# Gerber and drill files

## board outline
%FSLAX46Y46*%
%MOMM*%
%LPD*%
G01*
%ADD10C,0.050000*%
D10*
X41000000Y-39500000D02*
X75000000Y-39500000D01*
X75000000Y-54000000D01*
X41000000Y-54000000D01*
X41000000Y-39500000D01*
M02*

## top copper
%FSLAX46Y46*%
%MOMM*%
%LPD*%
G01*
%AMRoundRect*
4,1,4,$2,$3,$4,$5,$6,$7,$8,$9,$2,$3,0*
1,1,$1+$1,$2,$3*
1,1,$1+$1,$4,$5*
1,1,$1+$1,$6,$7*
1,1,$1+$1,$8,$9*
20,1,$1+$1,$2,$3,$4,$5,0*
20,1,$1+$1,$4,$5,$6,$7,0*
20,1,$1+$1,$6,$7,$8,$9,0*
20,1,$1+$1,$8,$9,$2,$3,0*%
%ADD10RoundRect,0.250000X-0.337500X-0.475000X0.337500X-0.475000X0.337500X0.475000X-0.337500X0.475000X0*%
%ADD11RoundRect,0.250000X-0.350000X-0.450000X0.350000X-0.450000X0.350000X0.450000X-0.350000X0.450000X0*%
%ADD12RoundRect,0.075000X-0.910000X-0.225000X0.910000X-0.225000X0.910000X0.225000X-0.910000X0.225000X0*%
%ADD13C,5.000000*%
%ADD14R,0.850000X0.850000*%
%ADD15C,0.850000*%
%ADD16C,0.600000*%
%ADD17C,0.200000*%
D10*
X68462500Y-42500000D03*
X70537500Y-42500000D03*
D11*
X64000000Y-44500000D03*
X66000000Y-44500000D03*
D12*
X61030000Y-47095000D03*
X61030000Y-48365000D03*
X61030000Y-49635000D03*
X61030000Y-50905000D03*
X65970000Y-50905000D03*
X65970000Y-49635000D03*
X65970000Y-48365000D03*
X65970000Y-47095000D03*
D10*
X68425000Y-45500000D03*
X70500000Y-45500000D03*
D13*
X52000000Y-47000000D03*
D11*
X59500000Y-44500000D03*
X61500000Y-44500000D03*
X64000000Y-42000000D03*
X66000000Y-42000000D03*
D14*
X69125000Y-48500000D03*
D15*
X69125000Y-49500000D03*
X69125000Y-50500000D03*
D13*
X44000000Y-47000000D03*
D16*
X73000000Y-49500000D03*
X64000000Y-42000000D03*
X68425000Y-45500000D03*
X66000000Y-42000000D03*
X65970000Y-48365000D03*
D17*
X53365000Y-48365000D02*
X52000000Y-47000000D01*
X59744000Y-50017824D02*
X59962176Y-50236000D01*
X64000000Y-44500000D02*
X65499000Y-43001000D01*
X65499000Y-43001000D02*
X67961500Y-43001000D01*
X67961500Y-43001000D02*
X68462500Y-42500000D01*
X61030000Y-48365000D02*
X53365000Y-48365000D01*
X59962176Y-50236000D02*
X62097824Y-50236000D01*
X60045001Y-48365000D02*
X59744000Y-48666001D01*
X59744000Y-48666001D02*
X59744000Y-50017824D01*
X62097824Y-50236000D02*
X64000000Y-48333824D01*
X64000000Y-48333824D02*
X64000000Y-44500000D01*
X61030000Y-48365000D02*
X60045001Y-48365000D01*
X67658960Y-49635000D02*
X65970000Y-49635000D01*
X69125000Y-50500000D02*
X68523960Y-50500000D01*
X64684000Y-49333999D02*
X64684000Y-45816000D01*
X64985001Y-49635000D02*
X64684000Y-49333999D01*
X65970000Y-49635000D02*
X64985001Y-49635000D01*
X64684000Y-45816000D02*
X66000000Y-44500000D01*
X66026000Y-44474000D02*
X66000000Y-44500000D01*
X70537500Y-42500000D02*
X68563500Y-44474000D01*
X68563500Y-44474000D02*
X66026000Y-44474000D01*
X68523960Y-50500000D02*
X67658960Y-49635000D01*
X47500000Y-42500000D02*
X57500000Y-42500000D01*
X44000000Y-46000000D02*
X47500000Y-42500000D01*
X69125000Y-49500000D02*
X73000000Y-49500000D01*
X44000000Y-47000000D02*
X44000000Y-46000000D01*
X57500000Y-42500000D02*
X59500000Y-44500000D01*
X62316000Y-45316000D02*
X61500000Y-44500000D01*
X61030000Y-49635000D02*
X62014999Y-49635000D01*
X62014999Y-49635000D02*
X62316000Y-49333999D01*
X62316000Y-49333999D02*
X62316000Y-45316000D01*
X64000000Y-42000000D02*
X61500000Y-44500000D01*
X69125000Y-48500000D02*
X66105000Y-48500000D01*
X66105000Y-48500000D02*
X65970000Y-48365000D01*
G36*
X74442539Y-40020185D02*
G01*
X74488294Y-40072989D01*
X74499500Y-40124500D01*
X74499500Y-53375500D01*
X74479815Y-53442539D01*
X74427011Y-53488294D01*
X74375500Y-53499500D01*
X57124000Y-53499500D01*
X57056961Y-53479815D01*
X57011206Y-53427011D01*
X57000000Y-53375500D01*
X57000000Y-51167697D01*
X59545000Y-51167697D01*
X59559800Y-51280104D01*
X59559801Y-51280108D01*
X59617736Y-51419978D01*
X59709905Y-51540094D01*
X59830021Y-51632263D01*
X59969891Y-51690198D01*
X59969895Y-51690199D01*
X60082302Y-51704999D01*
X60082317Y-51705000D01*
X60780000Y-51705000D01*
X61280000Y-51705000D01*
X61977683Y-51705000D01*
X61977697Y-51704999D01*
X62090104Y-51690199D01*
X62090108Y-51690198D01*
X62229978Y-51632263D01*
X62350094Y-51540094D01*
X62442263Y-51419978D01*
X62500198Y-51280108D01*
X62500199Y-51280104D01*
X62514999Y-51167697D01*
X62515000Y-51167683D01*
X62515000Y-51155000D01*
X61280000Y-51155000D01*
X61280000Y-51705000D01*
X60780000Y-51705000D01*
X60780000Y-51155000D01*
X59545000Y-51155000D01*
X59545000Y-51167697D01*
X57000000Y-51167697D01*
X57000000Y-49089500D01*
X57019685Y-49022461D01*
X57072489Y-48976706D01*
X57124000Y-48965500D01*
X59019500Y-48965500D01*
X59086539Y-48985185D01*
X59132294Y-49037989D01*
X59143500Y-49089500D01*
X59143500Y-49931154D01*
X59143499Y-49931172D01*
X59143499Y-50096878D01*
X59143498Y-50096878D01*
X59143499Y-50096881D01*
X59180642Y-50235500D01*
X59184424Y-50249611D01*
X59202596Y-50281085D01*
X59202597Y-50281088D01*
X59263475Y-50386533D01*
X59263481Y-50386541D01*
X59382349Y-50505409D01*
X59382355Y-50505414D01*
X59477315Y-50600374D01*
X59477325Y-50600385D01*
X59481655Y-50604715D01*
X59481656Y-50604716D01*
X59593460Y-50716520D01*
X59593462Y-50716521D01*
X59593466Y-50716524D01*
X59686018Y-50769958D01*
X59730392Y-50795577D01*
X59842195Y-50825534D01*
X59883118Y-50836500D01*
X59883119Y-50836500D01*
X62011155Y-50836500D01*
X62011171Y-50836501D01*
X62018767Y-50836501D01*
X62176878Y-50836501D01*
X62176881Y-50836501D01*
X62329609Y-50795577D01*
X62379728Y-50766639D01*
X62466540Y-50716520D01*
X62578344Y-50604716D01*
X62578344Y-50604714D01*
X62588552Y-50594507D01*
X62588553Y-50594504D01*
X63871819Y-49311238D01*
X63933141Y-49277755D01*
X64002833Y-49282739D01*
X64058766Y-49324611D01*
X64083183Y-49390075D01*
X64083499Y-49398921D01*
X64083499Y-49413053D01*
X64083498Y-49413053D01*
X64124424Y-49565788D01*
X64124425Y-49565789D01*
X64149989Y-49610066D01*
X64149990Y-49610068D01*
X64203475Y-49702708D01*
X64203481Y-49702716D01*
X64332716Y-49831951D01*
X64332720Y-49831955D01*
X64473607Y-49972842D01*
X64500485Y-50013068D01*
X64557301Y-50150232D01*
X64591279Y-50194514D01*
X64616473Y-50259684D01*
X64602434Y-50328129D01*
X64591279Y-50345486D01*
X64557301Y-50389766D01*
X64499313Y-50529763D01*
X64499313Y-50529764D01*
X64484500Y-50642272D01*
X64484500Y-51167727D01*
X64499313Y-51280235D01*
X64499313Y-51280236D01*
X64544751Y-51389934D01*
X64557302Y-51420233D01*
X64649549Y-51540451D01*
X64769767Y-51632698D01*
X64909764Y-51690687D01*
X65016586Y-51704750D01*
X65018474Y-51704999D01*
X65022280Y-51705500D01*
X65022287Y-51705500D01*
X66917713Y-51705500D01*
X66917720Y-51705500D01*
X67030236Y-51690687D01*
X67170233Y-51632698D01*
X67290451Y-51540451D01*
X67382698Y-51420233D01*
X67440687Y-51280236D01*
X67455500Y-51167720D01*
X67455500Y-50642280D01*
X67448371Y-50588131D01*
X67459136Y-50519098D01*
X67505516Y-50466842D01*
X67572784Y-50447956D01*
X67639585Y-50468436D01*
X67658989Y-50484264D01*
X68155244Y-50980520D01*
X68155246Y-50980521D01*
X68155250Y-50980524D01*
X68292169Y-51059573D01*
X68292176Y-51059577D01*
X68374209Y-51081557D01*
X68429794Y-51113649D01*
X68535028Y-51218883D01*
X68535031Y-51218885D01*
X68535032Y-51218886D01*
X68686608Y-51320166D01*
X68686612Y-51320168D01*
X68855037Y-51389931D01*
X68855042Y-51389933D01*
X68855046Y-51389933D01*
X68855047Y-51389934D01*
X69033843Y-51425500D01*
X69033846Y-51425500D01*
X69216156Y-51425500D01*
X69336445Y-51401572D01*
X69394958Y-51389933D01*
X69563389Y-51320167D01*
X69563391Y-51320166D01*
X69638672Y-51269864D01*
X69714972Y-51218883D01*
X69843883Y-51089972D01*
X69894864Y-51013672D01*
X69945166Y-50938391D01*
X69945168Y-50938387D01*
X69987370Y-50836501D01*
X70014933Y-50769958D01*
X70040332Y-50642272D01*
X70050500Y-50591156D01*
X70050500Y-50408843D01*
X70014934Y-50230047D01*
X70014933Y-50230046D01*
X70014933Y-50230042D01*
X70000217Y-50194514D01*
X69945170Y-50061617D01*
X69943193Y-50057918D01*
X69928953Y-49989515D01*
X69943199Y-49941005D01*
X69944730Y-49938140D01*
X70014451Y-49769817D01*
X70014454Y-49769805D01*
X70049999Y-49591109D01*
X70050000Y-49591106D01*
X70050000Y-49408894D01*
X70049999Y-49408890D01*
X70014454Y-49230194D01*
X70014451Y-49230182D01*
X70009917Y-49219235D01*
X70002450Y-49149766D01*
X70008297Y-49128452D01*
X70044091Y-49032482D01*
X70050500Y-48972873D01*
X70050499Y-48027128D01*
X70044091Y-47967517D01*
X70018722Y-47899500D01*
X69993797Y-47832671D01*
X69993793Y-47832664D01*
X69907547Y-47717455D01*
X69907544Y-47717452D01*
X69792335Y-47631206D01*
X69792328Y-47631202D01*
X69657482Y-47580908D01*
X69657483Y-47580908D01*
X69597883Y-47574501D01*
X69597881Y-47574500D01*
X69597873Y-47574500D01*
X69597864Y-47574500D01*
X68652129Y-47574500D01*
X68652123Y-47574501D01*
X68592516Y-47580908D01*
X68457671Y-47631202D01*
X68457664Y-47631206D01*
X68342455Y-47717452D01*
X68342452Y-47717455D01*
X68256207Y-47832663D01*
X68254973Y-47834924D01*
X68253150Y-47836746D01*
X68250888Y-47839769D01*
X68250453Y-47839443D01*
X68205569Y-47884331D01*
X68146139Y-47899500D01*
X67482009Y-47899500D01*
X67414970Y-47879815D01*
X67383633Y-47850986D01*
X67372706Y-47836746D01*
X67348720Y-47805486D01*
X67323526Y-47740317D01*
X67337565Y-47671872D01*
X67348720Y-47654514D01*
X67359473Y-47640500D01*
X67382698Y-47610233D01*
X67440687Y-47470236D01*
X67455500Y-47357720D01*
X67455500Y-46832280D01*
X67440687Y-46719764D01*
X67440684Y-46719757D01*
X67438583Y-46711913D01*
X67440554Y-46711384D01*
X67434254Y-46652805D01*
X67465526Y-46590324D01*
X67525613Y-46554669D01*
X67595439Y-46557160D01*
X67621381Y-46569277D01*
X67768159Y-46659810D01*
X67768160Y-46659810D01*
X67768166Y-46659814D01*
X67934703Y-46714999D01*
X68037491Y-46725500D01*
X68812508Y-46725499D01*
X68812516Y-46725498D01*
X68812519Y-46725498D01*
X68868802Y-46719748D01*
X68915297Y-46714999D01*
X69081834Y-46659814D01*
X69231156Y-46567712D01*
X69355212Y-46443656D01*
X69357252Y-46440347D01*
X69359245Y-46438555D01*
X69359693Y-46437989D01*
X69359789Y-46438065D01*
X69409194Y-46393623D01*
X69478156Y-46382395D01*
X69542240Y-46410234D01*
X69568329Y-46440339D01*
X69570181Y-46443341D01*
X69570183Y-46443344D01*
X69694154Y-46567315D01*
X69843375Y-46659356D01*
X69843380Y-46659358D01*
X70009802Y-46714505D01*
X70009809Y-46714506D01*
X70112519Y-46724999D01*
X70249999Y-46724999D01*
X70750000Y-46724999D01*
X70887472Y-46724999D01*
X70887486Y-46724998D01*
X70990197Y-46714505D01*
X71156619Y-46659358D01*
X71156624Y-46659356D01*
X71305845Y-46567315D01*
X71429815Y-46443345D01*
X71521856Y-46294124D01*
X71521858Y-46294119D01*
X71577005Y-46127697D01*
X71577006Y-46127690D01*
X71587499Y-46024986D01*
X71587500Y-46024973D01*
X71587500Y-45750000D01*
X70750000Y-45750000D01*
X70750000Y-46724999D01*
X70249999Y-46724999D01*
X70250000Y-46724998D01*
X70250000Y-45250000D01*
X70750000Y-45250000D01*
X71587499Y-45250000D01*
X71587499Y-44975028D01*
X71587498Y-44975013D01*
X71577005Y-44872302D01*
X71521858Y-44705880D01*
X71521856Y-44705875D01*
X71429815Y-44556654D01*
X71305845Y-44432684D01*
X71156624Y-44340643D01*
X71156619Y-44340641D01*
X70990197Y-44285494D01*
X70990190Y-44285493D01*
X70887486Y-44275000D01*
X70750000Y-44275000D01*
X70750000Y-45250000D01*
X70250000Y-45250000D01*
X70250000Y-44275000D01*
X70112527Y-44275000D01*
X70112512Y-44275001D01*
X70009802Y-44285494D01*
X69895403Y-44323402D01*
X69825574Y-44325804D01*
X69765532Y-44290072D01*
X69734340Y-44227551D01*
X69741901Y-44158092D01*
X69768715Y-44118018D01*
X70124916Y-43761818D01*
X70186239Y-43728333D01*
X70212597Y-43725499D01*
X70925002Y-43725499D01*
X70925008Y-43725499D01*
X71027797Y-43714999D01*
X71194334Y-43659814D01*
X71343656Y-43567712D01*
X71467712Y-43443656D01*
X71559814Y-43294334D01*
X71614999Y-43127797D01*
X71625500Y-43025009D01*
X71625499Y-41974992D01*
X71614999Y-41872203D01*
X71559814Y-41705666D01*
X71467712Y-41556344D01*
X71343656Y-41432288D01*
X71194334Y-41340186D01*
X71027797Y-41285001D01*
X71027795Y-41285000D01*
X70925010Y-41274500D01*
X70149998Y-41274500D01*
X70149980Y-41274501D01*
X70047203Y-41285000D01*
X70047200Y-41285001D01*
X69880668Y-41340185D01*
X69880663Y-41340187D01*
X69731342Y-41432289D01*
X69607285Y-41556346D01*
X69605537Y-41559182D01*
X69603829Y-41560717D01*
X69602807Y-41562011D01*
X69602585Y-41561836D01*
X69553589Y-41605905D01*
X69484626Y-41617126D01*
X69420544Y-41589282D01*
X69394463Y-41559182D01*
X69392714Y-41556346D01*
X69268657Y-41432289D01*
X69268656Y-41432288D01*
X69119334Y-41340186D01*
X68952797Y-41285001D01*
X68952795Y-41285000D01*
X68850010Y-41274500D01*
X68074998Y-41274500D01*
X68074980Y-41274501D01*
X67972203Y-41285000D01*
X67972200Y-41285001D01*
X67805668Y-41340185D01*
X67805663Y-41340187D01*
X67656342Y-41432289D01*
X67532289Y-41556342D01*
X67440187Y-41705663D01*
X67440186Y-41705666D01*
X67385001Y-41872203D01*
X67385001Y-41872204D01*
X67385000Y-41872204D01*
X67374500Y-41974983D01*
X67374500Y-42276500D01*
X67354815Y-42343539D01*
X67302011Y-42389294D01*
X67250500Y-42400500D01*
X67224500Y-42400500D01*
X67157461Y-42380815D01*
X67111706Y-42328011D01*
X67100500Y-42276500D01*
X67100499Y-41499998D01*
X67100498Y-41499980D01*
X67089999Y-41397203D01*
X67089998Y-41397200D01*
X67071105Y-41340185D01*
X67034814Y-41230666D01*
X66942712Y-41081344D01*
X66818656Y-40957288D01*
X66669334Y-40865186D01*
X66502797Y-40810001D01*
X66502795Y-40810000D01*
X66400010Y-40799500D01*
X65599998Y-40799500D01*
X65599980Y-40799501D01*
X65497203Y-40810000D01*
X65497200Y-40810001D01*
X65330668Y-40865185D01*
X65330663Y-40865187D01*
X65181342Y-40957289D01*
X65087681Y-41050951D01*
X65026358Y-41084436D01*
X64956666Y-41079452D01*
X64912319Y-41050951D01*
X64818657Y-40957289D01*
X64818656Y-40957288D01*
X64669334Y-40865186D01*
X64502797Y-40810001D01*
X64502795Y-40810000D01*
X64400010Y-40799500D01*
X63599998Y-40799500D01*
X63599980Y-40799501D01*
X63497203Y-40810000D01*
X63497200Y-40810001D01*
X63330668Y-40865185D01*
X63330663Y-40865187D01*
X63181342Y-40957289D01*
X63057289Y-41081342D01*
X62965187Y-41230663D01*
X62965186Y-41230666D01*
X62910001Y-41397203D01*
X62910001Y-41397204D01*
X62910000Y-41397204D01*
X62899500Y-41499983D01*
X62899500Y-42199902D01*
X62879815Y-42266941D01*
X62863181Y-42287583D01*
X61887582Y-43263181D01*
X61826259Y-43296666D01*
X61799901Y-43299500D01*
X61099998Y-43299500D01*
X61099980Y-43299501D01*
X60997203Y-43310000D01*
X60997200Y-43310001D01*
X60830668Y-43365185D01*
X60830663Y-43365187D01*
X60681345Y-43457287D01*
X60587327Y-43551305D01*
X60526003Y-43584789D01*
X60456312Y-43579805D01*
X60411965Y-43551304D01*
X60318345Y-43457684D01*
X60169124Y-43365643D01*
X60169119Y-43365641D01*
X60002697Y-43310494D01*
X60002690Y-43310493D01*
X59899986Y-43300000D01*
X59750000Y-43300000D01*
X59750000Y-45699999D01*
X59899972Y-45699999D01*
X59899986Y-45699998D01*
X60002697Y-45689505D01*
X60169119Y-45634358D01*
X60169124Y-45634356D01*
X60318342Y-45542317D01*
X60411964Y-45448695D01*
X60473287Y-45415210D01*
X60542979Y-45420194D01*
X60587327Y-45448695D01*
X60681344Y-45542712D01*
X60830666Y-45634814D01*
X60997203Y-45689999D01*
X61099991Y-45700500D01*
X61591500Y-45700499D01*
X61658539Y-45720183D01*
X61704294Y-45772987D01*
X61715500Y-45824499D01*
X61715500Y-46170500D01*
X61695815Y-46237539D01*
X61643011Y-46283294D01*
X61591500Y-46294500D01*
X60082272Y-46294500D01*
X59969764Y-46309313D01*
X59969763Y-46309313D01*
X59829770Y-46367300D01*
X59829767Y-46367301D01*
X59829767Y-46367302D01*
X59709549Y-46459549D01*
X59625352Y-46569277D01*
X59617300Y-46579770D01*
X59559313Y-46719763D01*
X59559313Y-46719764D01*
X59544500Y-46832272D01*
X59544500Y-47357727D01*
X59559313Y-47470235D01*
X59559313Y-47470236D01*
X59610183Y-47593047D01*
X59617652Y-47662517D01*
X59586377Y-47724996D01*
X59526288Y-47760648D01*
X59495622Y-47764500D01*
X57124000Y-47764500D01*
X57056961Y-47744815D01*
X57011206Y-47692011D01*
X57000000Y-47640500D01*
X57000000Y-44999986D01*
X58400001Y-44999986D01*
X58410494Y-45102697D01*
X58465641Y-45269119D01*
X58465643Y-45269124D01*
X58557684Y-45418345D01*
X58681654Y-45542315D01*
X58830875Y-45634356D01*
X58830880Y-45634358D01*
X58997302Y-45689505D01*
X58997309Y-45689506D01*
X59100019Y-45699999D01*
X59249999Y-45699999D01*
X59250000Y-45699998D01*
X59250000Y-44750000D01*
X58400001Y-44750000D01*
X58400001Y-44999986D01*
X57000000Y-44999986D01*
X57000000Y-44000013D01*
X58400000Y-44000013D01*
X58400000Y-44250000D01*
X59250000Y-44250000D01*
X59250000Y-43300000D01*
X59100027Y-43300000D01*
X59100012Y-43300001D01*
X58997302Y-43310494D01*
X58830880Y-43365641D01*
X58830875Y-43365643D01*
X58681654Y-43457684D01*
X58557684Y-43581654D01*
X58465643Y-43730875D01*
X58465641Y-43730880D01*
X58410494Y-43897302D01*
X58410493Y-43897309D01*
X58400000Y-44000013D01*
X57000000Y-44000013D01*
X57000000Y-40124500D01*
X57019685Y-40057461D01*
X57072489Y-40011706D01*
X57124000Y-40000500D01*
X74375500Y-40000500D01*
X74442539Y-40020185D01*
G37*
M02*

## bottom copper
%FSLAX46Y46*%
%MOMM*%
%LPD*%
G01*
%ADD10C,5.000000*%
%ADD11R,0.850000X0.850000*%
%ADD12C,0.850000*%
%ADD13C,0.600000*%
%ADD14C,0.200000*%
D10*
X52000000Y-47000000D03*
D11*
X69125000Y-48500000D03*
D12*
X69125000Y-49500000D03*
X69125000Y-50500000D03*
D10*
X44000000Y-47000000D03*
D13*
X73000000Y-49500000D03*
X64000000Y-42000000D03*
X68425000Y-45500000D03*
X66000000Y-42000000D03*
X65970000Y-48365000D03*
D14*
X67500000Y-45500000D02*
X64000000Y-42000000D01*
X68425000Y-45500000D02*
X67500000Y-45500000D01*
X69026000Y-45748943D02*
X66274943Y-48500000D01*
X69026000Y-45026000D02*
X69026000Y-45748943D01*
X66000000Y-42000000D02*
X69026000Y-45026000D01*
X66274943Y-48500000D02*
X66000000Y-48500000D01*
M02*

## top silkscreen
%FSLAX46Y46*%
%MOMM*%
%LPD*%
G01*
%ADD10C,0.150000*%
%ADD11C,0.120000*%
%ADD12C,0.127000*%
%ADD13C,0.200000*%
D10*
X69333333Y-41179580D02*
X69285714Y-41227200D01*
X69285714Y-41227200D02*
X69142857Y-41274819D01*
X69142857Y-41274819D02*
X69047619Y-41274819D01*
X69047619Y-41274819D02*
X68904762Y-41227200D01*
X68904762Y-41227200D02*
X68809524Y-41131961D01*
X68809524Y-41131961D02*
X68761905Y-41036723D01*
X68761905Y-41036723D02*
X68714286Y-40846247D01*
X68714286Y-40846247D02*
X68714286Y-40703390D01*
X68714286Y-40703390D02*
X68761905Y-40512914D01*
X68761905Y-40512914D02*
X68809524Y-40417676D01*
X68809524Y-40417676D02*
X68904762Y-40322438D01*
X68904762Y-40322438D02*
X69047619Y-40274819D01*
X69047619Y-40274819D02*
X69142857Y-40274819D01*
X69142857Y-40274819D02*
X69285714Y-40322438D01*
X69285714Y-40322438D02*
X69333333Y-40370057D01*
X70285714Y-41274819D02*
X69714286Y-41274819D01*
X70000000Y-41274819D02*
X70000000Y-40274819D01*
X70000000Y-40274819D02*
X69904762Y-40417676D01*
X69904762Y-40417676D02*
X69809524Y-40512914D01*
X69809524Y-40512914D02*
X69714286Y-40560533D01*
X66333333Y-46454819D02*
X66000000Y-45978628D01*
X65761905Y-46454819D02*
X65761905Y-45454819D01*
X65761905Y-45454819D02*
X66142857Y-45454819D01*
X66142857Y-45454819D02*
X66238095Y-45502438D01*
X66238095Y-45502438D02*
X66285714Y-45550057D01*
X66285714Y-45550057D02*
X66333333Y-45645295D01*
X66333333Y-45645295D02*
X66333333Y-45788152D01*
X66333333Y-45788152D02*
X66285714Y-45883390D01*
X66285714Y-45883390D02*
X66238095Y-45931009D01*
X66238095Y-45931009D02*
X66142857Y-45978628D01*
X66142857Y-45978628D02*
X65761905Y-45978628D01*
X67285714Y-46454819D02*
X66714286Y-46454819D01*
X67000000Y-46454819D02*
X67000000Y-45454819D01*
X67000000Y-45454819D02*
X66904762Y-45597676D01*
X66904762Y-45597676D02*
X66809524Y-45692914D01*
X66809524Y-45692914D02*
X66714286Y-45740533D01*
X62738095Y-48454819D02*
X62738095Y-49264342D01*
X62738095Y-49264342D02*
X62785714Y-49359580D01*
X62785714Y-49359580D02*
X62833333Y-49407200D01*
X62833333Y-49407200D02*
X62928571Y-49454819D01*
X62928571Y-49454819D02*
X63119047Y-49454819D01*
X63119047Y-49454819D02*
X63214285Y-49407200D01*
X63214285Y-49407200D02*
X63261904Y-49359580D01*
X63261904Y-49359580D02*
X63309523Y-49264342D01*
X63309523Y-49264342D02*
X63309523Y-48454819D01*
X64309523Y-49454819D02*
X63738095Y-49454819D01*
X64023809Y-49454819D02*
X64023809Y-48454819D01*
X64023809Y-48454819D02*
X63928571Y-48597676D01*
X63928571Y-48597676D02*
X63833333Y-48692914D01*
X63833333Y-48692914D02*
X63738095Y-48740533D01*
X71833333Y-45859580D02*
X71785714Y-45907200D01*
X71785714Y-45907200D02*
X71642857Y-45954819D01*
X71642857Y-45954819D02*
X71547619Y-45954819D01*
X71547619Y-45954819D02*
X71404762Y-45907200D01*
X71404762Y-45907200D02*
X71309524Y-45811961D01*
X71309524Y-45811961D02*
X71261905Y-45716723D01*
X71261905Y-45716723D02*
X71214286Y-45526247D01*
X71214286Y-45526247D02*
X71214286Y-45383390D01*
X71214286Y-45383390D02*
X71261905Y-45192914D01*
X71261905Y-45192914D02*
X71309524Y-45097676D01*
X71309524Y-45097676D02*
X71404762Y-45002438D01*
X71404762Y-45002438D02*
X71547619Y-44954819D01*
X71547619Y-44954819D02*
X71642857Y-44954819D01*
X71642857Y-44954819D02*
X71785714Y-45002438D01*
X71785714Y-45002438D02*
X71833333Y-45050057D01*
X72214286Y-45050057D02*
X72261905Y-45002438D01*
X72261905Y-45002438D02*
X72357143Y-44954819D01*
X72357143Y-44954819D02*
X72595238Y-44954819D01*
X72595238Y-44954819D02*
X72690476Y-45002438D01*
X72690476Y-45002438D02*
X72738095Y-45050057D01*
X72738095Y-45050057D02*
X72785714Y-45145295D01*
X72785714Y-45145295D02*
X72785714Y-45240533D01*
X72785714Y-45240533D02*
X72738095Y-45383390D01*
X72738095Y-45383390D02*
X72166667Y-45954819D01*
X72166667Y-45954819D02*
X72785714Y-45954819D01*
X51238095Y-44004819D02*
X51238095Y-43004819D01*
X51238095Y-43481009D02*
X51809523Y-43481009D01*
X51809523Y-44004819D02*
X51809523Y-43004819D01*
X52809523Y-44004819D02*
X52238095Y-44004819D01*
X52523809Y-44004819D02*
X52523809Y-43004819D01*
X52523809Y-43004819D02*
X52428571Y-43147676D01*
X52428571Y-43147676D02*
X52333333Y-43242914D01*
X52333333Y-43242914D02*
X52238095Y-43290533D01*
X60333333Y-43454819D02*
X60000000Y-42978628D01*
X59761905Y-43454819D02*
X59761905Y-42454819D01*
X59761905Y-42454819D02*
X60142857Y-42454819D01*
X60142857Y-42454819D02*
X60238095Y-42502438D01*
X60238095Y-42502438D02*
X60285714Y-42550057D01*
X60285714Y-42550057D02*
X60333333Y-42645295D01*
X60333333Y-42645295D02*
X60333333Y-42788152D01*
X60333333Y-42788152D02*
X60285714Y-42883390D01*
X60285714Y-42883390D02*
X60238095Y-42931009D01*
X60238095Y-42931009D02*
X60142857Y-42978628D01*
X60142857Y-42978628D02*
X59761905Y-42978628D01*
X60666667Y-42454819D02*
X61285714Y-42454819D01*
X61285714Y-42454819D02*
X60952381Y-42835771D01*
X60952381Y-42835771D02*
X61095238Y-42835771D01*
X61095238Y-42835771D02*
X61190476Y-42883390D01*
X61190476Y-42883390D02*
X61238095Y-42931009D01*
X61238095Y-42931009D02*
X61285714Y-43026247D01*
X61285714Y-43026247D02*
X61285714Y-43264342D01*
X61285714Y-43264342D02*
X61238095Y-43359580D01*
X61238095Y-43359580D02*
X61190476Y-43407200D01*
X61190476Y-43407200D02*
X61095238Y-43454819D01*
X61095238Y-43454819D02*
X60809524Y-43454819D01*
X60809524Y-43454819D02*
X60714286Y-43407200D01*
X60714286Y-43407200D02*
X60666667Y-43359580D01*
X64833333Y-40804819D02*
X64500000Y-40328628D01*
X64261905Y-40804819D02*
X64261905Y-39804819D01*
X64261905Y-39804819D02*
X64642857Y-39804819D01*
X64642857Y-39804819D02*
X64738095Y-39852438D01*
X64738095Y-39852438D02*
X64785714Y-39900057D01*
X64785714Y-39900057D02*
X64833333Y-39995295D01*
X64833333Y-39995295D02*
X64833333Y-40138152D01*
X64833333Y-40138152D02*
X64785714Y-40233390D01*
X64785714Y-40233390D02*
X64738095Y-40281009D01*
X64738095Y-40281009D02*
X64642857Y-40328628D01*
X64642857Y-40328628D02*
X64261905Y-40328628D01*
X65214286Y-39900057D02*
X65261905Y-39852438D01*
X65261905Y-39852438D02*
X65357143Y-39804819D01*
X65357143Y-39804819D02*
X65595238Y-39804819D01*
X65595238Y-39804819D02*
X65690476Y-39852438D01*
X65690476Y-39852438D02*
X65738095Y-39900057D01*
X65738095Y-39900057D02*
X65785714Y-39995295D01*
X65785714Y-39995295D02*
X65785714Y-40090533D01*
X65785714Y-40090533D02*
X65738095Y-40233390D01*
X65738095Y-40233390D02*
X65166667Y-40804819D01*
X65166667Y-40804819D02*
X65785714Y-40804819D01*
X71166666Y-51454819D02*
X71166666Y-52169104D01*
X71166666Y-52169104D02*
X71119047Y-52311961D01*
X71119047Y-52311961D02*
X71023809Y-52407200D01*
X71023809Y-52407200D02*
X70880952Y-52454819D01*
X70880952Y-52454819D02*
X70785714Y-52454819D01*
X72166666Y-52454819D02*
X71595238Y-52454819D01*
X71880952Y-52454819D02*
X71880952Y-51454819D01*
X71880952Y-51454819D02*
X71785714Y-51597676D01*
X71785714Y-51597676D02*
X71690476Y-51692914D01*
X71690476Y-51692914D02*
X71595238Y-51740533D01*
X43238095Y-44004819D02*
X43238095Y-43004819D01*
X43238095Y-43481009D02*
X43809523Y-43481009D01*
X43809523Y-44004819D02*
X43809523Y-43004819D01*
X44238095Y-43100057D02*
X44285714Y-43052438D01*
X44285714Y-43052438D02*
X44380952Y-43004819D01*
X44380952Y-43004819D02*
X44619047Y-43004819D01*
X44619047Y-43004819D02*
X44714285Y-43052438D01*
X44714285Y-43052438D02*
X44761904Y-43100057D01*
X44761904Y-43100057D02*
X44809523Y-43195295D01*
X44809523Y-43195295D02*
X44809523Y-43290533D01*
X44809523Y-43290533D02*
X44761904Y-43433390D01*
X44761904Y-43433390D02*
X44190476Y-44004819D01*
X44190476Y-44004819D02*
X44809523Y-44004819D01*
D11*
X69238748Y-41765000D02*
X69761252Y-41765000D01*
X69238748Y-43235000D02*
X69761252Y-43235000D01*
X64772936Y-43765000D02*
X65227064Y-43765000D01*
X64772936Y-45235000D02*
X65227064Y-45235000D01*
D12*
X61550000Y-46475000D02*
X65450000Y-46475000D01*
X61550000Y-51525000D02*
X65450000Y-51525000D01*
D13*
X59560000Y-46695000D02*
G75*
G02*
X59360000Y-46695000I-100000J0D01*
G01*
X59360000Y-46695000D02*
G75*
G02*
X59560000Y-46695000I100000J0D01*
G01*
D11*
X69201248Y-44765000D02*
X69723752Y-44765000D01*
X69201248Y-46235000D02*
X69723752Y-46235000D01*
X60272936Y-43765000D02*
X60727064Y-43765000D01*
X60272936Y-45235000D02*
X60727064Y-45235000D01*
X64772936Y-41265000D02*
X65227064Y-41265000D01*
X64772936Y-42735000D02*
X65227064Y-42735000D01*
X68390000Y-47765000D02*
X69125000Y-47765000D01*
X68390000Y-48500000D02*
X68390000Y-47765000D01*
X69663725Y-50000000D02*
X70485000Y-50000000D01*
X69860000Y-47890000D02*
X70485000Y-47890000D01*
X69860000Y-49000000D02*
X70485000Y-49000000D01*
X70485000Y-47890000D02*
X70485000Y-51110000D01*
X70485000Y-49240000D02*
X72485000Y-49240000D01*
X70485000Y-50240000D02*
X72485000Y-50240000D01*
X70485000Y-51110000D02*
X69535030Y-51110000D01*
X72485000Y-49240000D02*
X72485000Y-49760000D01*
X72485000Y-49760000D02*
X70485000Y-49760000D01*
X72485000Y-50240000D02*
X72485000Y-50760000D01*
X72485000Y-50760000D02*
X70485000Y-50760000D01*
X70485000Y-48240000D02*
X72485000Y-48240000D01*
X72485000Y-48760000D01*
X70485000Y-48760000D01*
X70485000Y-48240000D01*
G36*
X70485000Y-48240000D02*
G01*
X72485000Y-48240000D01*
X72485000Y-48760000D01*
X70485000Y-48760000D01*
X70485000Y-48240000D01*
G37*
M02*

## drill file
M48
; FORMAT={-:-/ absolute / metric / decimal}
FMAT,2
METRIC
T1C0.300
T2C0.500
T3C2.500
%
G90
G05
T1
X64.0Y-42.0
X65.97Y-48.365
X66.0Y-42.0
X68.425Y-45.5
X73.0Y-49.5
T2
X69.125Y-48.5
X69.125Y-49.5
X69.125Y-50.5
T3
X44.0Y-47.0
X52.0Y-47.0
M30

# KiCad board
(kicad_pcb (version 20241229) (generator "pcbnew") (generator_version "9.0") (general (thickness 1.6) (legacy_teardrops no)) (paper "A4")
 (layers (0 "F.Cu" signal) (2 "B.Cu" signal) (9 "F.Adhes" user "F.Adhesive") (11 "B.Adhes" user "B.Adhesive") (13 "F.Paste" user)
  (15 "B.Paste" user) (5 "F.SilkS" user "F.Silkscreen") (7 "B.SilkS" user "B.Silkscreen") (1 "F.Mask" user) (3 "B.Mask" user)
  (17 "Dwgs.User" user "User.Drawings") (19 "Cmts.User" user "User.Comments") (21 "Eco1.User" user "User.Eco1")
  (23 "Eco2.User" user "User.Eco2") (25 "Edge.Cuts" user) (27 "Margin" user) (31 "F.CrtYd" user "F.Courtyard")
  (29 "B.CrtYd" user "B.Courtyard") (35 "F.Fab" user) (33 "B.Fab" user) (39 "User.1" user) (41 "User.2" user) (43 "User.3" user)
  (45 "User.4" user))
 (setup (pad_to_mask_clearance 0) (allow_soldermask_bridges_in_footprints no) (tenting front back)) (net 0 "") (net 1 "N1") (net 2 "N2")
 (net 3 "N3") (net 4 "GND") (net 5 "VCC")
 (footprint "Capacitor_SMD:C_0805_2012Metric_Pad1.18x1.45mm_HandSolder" (layer "F.Cu") (at 69.5 42.5)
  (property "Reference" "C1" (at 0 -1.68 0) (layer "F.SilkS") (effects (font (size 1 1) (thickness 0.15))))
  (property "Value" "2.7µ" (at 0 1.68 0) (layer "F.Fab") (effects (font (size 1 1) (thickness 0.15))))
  (fp_line (start -0.261252 -0.735) (end 0.261252 -0.735) (stroke (width 0.12) (type solid)) (layer "F.SilkS"))
  (fp_line (start -0.261252 0.735) (end 0.261252 0.735) (stroke (width 0.12) (type solid)) (layer "F.SilkS"))
  (pad "1" smd roundrect (at -1.0375 0) (size 1.175 1.45) (layers "F.Cu" "F.Mask" "F.Paste") (roundrect_rratio 0.212766) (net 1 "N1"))
  (pad "2" smd roundrect (at 1.0375 0) (size 1.175 1.45) (layers "F.Cu" "F.Mask" "F.Paste") (roundrect_rratio 0.212766) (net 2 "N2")))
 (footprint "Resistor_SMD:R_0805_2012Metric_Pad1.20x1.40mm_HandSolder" (layer "F.Cu") (at 65 44.5)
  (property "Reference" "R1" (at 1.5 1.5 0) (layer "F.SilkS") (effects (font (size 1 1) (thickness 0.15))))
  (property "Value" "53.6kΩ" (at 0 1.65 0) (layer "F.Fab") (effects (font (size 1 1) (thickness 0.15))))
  (fp_line (start -0.227064 -0.735) (end 0.227064 -0.735) (stroke (width 0.12) (type solid)) (layer "F.SilkS"))
  (fp_line (start -0.227064 0.735) (end 0.227064 0.735) (stroke (width 0.12) (type solid)) (layer "F.SilkS"))
  (pad "1" smd roundrect (at -1 0) (size 1.2 1.4) (layers "F.Cu" "F.Mask" "F.Paste") (roundrect_rratio 0.208333) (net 1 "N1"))
  (pad "2" smd roundrect (at 1 0) (size 1.2 1.4) (layers "F.Cu" "F.Mask" "F.Paste") (roundrect_rratio 0.208333) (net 2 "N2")))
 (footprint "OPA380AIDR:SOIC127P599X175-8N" (layer "F.Cu") (at 63.5 49)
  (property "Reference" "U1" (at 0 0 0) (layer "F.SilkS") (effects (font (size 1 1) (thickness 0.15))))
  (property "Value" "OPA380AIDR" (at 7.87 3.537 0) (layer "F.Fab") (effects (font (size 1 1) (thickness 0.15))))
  (fp_line (start -1.95 -2.525) (end 1.95 -2.525) (stroke (width 0.127) (type solid)) (layer "F.SilkS"))
  (fp_line (start -1.95 2.525) (end 1.95 2.525) (stroke (width 0.127) (type solid)) (layer "F.SilkS"))
  (fp_circle (center -4.04 -2.305) (end -3.94 -2.305) (stroke (width 0.2) (type solid)) (fill no) (layer "F.SilkS"))
  (pad "1" smd roundrect (at -2.47 -1.905) (size 1.97 0.6) (layers "F.Cu" "F.Mask" "F.Paste") (roundrect_rratio 0.125)
   (solder_mask_margin 0.102))
  (pad "2" smd roundrect (at -2.47 -0.635) (size 1.97 0.6) (layers "F.Cu" "F.Mask" "F.Paste") (roundrect_rratio 0.125) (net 1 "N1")
   (solder_mask_margin 0.102))
  (pad "3" smd roundrect (at -2.47 0.635) (size 1.97 0.6) (layers "F.Cu" "F.Mask" "F.Paste") (roundrect_rratio 0.125) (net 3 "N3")
   (solder_mask_margin 0.102))
  (pad "4" smd roundrect (at -2.47 1.905) (size 1.97 0.6) (layers "F.Cu" "F.Mask" "F.Paste") (roundrect_rratio 0.125) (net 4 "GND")
   (solder_mask_margin 0.102))
  (pad "5" smd roundrect (at 2.47 1.905) (size 1.97 0.6) (layers "F.Cu" "F.Mask" "F.Paste") (roundrect_rratio 0.125)
   (solder_mask_margin 0.102))
  (pad "6" smd roundrect (at 2.47 0.635) (size 1.97 0.6) (layers "F.Cu" "F.Mask" "F.Paste") (roundrect_rratio 0.125) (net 2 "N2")
   (solder_mask_margin 0.102))
  (pad "7" smd roundrect (at 2.47 -0.635) (size 1.97 0.6) (layers "F.Cu" "F.Mask" "F.Paste") (roundrect_rratio 0.125) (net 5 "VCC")
   (solder_mask_margin 0.102))
  (pad "8" smd roundrect (at 2.47 -1.905) (size 1.97 0.6) (layers "F.Cu" "F.Mask" "F.Paste") (roundrect_rratio 0.125)
   (solder_mask_margin 0.102)))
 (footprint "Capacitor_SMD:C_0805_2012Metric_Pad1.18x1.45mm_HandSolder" (layer "F.Cu") (at 69.4625 45.5)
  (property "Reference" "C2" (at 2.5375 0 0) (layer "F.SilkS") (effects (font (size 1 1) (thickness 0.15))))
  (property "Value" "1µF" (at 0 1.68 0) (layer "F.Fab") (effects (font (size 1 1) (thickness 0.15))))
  (fp_line (start -0.261252 -0.735) (end 0.261252 -0.735) (stroke (width 0.12) (type solid)) (layer "F.SilkS"))
  (fp_line (start -0.261252 0.735) (end 0.261252 0.735) (stroke (width 0.12) (type solid)) (layer "F.SilkS"))
  (pad "1" smd roundrect (at -1.0375 0) (size 1.175 1.45) (layers "F.Cu" "F.Mask" "F.Paste") (roundrect_rratio 0.212766) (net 3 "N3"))
  (pad "2" smd roundrect (at 1.0375 0) (size 1.175 1.45) (layers "F.Cu" "F.Mask" "F.Paste") (roundrect_rratio 0.212766) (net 4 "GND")))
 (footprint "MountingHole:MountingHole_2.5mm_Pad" (layer "F.Cu") (at 52 47)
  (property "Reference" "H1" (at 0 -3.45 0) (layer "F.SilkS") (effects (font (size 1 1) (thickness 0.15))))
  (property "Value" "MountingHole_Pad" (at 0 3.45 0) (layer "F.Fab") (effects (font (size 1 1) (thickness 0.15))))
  (pad "1" thru_hole circle (at 0 0) (size 5 5) (drill 2.5) (layers "*.Cu" "*.Mask") (remove_unused_layers no) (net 1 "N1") (zone_connect 2)))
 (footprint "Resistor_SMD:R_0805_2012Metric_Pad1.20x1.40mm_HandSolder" (layer "F.Cu") (at 60.5 44.5)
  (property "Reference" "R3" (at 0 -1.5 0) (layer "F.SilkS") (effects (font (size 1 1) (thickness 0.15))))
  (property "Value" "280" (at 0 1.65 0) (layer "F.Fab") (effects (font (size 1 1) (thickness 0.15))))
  (fp_line (start -0.227064 -0.735) (end 0.227064 -0.735) (stroke (width 0.12) (type solid)) (layer "F.SilkS"))
  (fp_line (start -0.227064 0.735) (end 0.227064 0.735) (stroke (width 0.12) (type solid)) (layer "F.SilkS"))
  (pad "1" smd roundrect (at -1 0) (size 1.2 1.4) (layers "F.Cu" "F.Mask" "F.Paste") (roundrect_rratio 0.208333) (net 4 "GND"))
  (pad "2" smd roundrect (at 1 0) (size 1.2 1.4) (layers "F.Cu" "F.Mask" "F.Paste") (roundrect_rratio 0.208333) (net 3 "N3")))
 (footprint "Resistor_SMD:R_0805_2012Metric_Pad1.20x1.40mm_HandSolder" (layer "F.Cu") (at 65 42)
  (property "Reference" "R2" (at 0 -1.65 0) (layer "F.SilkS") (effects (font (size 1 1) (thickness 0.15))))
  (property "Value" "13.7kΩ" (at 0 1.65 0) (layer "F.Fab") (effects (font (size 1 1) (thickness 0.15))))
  (fp_line (start -0.227064 -0.735) (end 0.227064 -0.735) (stroke (width 0.12) (type solid)) (layer "F.SilkS"))
  (fp_line (start -0.227064 0.735) (end 0.227064 0.735) (stroke (width 0.12) (type solid)) (layer "F.SilkS"))
  (pad "1" smd roundrect (at -1 0) (size 1.2 1.4) (layers "F.Cu" "F.Mask" "F.Paste") (roundrect_rratio 0.208333) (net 3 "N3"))
  (pad "2" smd roundrect (at 1 0) (size 1.2 1.4) (layers "F.Cu" "F.Mask" "F.Paste") (roundrect_rratio 0.208333) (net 5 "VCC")))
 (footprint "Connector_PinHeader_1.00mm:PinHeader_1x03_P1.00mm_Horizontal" (layer "F.Cu") (at 69.125 48.5)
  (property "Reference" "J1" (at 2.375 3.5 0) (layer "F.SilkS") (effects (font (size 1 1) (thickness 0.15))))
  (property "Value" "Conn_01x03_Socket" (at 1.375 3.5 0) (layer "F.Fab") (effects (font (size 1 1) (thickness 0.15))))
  (fp_line (start -0.735 -0.735) (end 0 -0.735) (stroke (width 0.12) (type solid)) (layer "F.SilkS"))
  (fp_line (start -0.735 0) (end -0.735 -0.735) (stroke (width 0.12) (type solid)) (layer "F.SilkS"))
  (fp_line (start 0.538725 1.5) (end 1.36 1.5) (stroke (width 0.12) (type solid)) (layer "F.SilkS"))
  (fp_line (start 0.735 -0.61) (end 1.36 -0.61) (stroke (width 0.12) (type solid)) (layer "F.SilkS"))
  (fp_line (start 0.735 0.5) (end 1.36 0.5) (stroke (width 0.12) (type solid)) (layer "F.SilkS"))
  (fp_line (start 1.36 -0.61) (end 1.36 2.61) (stroke (width 0.12) (type solid)) (layer "F.SilkS"))
  (fp_line (start 1.36 0.74) (end 3.36 0.74) (stroke (width 0.12) (type solid)) (layer "F.SilkS"))
  (fp_line (start 1.36 1.74) (end 3.36 1.74) (stroke (width 0.12) (type solid)) (layer "F.SilkS"))
  (fp_line (start 1.36 2.61) (end 0.41003 2.61) (stroke (width 0.12) (type solid)) (layer "F.SilkS"))
  (fp_line (start 3.36 0.74) (end 3.36 1.26) (stroke (width 0.12) (type solid)) (layer "F.SilkS"))
  (fp_line (start 3.36 1.26) (end 1.36 1.26) (stroke (width 0.12) (type solid)) (layer "F.SilkS"))
  (fp_line (start 3.36 1.74) (end 3.36 2.26) (stroke (width 0.12) (type solid)) (layer "F.SilkS"))
  (fp_line (start 3.36 2.26) (end 1.36 2.26) (stroke (width 0.12) (type solid)) (layer "F.SilkS"))
  (fp_rect (start 1.36 -0.26) (end 3.36 0.26) (stroke (width 0.12) (type solid)) (fill yes) (layer "F.SilkS"))
  (pad "1" thru_hole rect (at 0 0) (size 0.85 0.85) (drill 0.5) (layers "*.Cu" "*.Mask") (remove_unused_layers no) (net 5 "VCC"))
  (pad "2" thru_hole circle (at 0 1) (size 0.85 0.85) (drill 0.5) (layers "*.Cu" "*.Mask") (remove_unused_layers no) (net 4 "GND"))
  (pad "3" thru_hole circle (at 0 2) (size 0.85 0.85) (drill 0.5) (layers "*.Cu" "*.Mask") (remove_unused_layers no) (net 2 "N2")))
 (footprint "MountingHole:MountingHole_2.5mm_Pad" (layer "F.Cu") (at 44 47)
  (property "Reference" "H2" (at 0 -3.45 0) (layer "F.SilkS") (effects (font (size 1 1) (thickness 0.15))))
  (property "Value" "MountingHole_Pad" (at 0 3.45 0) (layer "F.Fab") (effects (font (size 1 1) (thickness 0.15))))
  (pad "1" thru_hole circle (at 0 0) (size 5 5) (drill 2.5) (layers "*.Cu" "*.Mask") (remove_unused_layers no) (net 4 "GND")
   (zone_connect 2)))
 (gr_poly (pts (xy 41 39.5) (xy 75 39.5) (xy 75 54) (xy 41 54)) (stroke (width 0.05) (type solid)) (fill no) (layer "Edge.Cuts"))
 (segment (start 53.365 48.365) (end 52 47) (width 0.2) (layer "F.Cu") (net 1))
 (segment (start 59.744 50.017824) (end 59.962176 50.236) (width 0.2) (layer "F.Cu") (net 1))
 (segment (start 64 44.5) (end 65.499 43.001) (width 0.2) (layer "F.Cu") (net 1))
 (segment (start 65.499 43.001) (end 67.9615 43.001) (width 0.2) (layer "F.Cu") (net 1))
 (segment (start 67.9615 43.001) (end 68.4625 42.5) (width 0.2) (layer "F.Cu") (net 1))
 (segment (start 61.03 48.365) (end 53.365 48.365) (width 0.2) (layer "F.Cu") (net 1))
 (segment (start 59.962176 50.236) (end 62.097824 50.236) (width 0.2) (layer "F.Cu") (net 1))
 (segment (start 60.045001 48.365) (end 59.744 48.666001) (width 0.2) (layer "F.Cu") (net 1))
 (segment (start 59.744 48.666001) (end 59.744 50.017824) (width 0.2) (layer "F.Cu") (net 1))
 (segment (start 62.097824 50.236) (end 64 48.333824) (width 0.2) (layer "F.Cu") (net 1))
 (segment (start 64 48.333824) (end 64 44.5) (width 0.2) (layer "F.Cu") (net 1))
 (segment (start 61.03 48.365) (end 60.045001 48.365) (width 0.2) (layer "F.Cu") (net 1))
 (segment (start 67.65896 49.635) (end 65.97 49.635) (width 0.2) (layer "F.Cu") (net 2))
 (segment (start 69.125 50.5) (end 68.52396 50.5) (width 0.2) (layer "F.Cu") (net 2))
 (segment (start 64.684 49.333999) (end 64.684 45.816) (width 0.2) (layer "F.Cu") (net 2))
 (segment (start 64.985001 49.635) (end 64.684 49.333999) (width 0.2) (layer "F.Cu") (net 2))
 (segment (start 65.97 49.635) (end 64.985001 49.635) (width 0.2) (layer "F.Cu") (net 2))
 (segment (start 64.684 45.816) (end 66 44.5) (width 0.2) (layer "F.Cu") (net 2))
 (segment (start 66.026 44.474) (end 66 44.5) (width 0.2) (layer "F.Cu") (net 2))
 (segment (start 70.5375 42.5) (end 68.5635 44.474) (width 0.2) (layer "F.Cu") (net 2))
 (segment (start 68.5635 44.474) (end 66.026 44.474) (width 0.2) (layer "F.Cu") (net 2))
 (segment (start 68.52396 50.5) (end 67.65896 49.635) (width 0.2) (layer "F.Cu") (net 2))
 (segment (start 47.5 42.5) (end 57.5 42.5) (width 0.2) (layer "F.Cu") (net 4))
 (segment (start 44 46) (end 47.5 42.5) (width 0.2) (layer "F.Cu") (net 4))
 (segment (start 69.125 49.5) (end 73 49.5) (width 0.2) (layer "F.Cu") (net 4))
 (segment (start 44 47) (end 44 46) (width 0.2) (layer "F.Cu") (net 4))
 (segment (start 57.5 42.5) (end 59.5 44.5) (width 0.2) (layer "F.Cu") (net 4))
 (via (at 73 49.5) (size 0.6) (drill 0.3) (layers "F.Cu" "B.Cu") (free yes) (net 4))
 (segment (start 62.316 45.316) (end 61.5 44.5) (width 0.2) (layer "F.Cu") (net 3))
 (segment (start 61.03 49.635) (end 62.014999 49.635) (width 0.2) (layer "F.Cu") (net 3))
 (segment (start 62.014999 49.635) (end 62.316 49.333999) (width 0.2) (layer "F.Cu") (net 3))
 (segment (start 62.316 49.333999) (end 62.316 45.316) (width 0.2) (layer "F.Cu") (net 3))
 (segment (start 64 42) (end 61.5 44.5) (width 0.2) (layer "F.Cu") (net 3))
 (via (at 64 42) (size 0.6) (drill 0.3) (layers "F.Cu" "B.Cu") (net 3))
 (via (at 68.425 45.5) (size 0.6) (drill 0.3) (layers "F.Cu" "B.Cu") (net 3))
 (segment (start 67.5 45.5) (end 64 42) (width 0.2) (layer "B.Cu") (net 3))
 (segment (start 68.425 45.5) (end 67.5 45.5) (width 0.2) (layer "B.Cu") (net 3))
 (segment (start 69.125 48.5) (end 66.105 48.5) (width 0.2) (layer "F.Cu") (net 5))
 (segment (start 66.105 48.5) (end 65.97 48.365) (width 0.2) (layer "F.Cu") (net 5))
 (via (at 66 42) (size 0.6) (drill 0.3) (layers "F.Cu" "B.Cu") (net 5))
 (via (at 65.97 48.365) (size 0.6) (drill 0.3) (layers "F.Cu" "B.Cu") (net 5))
 (segment (start 69.026 45.748943) (end 66.274943 48.5) (width 0.2) (layer "B.Cu") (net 5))
 (segment (start 69.026 45.026) (end 69.026 45.748943) (width 0.2) (layer "B.Cu") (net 5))
 (segment (start 66 42) (end 69.026 45.026) (width 0.2) (layer "B.Cu") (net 5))
 (segment (start 66.274943 48.5) (end 66 48.5) (width 0.2) (layer "B.Cu") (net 5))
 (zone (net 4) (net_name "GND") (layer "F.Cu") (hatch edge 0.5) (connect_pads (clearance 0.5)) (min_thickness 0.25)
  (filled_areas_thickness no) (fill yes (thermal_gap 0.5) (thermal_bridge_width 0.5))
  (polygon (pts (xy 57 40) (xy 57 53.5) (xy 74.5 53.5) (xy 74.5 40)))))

